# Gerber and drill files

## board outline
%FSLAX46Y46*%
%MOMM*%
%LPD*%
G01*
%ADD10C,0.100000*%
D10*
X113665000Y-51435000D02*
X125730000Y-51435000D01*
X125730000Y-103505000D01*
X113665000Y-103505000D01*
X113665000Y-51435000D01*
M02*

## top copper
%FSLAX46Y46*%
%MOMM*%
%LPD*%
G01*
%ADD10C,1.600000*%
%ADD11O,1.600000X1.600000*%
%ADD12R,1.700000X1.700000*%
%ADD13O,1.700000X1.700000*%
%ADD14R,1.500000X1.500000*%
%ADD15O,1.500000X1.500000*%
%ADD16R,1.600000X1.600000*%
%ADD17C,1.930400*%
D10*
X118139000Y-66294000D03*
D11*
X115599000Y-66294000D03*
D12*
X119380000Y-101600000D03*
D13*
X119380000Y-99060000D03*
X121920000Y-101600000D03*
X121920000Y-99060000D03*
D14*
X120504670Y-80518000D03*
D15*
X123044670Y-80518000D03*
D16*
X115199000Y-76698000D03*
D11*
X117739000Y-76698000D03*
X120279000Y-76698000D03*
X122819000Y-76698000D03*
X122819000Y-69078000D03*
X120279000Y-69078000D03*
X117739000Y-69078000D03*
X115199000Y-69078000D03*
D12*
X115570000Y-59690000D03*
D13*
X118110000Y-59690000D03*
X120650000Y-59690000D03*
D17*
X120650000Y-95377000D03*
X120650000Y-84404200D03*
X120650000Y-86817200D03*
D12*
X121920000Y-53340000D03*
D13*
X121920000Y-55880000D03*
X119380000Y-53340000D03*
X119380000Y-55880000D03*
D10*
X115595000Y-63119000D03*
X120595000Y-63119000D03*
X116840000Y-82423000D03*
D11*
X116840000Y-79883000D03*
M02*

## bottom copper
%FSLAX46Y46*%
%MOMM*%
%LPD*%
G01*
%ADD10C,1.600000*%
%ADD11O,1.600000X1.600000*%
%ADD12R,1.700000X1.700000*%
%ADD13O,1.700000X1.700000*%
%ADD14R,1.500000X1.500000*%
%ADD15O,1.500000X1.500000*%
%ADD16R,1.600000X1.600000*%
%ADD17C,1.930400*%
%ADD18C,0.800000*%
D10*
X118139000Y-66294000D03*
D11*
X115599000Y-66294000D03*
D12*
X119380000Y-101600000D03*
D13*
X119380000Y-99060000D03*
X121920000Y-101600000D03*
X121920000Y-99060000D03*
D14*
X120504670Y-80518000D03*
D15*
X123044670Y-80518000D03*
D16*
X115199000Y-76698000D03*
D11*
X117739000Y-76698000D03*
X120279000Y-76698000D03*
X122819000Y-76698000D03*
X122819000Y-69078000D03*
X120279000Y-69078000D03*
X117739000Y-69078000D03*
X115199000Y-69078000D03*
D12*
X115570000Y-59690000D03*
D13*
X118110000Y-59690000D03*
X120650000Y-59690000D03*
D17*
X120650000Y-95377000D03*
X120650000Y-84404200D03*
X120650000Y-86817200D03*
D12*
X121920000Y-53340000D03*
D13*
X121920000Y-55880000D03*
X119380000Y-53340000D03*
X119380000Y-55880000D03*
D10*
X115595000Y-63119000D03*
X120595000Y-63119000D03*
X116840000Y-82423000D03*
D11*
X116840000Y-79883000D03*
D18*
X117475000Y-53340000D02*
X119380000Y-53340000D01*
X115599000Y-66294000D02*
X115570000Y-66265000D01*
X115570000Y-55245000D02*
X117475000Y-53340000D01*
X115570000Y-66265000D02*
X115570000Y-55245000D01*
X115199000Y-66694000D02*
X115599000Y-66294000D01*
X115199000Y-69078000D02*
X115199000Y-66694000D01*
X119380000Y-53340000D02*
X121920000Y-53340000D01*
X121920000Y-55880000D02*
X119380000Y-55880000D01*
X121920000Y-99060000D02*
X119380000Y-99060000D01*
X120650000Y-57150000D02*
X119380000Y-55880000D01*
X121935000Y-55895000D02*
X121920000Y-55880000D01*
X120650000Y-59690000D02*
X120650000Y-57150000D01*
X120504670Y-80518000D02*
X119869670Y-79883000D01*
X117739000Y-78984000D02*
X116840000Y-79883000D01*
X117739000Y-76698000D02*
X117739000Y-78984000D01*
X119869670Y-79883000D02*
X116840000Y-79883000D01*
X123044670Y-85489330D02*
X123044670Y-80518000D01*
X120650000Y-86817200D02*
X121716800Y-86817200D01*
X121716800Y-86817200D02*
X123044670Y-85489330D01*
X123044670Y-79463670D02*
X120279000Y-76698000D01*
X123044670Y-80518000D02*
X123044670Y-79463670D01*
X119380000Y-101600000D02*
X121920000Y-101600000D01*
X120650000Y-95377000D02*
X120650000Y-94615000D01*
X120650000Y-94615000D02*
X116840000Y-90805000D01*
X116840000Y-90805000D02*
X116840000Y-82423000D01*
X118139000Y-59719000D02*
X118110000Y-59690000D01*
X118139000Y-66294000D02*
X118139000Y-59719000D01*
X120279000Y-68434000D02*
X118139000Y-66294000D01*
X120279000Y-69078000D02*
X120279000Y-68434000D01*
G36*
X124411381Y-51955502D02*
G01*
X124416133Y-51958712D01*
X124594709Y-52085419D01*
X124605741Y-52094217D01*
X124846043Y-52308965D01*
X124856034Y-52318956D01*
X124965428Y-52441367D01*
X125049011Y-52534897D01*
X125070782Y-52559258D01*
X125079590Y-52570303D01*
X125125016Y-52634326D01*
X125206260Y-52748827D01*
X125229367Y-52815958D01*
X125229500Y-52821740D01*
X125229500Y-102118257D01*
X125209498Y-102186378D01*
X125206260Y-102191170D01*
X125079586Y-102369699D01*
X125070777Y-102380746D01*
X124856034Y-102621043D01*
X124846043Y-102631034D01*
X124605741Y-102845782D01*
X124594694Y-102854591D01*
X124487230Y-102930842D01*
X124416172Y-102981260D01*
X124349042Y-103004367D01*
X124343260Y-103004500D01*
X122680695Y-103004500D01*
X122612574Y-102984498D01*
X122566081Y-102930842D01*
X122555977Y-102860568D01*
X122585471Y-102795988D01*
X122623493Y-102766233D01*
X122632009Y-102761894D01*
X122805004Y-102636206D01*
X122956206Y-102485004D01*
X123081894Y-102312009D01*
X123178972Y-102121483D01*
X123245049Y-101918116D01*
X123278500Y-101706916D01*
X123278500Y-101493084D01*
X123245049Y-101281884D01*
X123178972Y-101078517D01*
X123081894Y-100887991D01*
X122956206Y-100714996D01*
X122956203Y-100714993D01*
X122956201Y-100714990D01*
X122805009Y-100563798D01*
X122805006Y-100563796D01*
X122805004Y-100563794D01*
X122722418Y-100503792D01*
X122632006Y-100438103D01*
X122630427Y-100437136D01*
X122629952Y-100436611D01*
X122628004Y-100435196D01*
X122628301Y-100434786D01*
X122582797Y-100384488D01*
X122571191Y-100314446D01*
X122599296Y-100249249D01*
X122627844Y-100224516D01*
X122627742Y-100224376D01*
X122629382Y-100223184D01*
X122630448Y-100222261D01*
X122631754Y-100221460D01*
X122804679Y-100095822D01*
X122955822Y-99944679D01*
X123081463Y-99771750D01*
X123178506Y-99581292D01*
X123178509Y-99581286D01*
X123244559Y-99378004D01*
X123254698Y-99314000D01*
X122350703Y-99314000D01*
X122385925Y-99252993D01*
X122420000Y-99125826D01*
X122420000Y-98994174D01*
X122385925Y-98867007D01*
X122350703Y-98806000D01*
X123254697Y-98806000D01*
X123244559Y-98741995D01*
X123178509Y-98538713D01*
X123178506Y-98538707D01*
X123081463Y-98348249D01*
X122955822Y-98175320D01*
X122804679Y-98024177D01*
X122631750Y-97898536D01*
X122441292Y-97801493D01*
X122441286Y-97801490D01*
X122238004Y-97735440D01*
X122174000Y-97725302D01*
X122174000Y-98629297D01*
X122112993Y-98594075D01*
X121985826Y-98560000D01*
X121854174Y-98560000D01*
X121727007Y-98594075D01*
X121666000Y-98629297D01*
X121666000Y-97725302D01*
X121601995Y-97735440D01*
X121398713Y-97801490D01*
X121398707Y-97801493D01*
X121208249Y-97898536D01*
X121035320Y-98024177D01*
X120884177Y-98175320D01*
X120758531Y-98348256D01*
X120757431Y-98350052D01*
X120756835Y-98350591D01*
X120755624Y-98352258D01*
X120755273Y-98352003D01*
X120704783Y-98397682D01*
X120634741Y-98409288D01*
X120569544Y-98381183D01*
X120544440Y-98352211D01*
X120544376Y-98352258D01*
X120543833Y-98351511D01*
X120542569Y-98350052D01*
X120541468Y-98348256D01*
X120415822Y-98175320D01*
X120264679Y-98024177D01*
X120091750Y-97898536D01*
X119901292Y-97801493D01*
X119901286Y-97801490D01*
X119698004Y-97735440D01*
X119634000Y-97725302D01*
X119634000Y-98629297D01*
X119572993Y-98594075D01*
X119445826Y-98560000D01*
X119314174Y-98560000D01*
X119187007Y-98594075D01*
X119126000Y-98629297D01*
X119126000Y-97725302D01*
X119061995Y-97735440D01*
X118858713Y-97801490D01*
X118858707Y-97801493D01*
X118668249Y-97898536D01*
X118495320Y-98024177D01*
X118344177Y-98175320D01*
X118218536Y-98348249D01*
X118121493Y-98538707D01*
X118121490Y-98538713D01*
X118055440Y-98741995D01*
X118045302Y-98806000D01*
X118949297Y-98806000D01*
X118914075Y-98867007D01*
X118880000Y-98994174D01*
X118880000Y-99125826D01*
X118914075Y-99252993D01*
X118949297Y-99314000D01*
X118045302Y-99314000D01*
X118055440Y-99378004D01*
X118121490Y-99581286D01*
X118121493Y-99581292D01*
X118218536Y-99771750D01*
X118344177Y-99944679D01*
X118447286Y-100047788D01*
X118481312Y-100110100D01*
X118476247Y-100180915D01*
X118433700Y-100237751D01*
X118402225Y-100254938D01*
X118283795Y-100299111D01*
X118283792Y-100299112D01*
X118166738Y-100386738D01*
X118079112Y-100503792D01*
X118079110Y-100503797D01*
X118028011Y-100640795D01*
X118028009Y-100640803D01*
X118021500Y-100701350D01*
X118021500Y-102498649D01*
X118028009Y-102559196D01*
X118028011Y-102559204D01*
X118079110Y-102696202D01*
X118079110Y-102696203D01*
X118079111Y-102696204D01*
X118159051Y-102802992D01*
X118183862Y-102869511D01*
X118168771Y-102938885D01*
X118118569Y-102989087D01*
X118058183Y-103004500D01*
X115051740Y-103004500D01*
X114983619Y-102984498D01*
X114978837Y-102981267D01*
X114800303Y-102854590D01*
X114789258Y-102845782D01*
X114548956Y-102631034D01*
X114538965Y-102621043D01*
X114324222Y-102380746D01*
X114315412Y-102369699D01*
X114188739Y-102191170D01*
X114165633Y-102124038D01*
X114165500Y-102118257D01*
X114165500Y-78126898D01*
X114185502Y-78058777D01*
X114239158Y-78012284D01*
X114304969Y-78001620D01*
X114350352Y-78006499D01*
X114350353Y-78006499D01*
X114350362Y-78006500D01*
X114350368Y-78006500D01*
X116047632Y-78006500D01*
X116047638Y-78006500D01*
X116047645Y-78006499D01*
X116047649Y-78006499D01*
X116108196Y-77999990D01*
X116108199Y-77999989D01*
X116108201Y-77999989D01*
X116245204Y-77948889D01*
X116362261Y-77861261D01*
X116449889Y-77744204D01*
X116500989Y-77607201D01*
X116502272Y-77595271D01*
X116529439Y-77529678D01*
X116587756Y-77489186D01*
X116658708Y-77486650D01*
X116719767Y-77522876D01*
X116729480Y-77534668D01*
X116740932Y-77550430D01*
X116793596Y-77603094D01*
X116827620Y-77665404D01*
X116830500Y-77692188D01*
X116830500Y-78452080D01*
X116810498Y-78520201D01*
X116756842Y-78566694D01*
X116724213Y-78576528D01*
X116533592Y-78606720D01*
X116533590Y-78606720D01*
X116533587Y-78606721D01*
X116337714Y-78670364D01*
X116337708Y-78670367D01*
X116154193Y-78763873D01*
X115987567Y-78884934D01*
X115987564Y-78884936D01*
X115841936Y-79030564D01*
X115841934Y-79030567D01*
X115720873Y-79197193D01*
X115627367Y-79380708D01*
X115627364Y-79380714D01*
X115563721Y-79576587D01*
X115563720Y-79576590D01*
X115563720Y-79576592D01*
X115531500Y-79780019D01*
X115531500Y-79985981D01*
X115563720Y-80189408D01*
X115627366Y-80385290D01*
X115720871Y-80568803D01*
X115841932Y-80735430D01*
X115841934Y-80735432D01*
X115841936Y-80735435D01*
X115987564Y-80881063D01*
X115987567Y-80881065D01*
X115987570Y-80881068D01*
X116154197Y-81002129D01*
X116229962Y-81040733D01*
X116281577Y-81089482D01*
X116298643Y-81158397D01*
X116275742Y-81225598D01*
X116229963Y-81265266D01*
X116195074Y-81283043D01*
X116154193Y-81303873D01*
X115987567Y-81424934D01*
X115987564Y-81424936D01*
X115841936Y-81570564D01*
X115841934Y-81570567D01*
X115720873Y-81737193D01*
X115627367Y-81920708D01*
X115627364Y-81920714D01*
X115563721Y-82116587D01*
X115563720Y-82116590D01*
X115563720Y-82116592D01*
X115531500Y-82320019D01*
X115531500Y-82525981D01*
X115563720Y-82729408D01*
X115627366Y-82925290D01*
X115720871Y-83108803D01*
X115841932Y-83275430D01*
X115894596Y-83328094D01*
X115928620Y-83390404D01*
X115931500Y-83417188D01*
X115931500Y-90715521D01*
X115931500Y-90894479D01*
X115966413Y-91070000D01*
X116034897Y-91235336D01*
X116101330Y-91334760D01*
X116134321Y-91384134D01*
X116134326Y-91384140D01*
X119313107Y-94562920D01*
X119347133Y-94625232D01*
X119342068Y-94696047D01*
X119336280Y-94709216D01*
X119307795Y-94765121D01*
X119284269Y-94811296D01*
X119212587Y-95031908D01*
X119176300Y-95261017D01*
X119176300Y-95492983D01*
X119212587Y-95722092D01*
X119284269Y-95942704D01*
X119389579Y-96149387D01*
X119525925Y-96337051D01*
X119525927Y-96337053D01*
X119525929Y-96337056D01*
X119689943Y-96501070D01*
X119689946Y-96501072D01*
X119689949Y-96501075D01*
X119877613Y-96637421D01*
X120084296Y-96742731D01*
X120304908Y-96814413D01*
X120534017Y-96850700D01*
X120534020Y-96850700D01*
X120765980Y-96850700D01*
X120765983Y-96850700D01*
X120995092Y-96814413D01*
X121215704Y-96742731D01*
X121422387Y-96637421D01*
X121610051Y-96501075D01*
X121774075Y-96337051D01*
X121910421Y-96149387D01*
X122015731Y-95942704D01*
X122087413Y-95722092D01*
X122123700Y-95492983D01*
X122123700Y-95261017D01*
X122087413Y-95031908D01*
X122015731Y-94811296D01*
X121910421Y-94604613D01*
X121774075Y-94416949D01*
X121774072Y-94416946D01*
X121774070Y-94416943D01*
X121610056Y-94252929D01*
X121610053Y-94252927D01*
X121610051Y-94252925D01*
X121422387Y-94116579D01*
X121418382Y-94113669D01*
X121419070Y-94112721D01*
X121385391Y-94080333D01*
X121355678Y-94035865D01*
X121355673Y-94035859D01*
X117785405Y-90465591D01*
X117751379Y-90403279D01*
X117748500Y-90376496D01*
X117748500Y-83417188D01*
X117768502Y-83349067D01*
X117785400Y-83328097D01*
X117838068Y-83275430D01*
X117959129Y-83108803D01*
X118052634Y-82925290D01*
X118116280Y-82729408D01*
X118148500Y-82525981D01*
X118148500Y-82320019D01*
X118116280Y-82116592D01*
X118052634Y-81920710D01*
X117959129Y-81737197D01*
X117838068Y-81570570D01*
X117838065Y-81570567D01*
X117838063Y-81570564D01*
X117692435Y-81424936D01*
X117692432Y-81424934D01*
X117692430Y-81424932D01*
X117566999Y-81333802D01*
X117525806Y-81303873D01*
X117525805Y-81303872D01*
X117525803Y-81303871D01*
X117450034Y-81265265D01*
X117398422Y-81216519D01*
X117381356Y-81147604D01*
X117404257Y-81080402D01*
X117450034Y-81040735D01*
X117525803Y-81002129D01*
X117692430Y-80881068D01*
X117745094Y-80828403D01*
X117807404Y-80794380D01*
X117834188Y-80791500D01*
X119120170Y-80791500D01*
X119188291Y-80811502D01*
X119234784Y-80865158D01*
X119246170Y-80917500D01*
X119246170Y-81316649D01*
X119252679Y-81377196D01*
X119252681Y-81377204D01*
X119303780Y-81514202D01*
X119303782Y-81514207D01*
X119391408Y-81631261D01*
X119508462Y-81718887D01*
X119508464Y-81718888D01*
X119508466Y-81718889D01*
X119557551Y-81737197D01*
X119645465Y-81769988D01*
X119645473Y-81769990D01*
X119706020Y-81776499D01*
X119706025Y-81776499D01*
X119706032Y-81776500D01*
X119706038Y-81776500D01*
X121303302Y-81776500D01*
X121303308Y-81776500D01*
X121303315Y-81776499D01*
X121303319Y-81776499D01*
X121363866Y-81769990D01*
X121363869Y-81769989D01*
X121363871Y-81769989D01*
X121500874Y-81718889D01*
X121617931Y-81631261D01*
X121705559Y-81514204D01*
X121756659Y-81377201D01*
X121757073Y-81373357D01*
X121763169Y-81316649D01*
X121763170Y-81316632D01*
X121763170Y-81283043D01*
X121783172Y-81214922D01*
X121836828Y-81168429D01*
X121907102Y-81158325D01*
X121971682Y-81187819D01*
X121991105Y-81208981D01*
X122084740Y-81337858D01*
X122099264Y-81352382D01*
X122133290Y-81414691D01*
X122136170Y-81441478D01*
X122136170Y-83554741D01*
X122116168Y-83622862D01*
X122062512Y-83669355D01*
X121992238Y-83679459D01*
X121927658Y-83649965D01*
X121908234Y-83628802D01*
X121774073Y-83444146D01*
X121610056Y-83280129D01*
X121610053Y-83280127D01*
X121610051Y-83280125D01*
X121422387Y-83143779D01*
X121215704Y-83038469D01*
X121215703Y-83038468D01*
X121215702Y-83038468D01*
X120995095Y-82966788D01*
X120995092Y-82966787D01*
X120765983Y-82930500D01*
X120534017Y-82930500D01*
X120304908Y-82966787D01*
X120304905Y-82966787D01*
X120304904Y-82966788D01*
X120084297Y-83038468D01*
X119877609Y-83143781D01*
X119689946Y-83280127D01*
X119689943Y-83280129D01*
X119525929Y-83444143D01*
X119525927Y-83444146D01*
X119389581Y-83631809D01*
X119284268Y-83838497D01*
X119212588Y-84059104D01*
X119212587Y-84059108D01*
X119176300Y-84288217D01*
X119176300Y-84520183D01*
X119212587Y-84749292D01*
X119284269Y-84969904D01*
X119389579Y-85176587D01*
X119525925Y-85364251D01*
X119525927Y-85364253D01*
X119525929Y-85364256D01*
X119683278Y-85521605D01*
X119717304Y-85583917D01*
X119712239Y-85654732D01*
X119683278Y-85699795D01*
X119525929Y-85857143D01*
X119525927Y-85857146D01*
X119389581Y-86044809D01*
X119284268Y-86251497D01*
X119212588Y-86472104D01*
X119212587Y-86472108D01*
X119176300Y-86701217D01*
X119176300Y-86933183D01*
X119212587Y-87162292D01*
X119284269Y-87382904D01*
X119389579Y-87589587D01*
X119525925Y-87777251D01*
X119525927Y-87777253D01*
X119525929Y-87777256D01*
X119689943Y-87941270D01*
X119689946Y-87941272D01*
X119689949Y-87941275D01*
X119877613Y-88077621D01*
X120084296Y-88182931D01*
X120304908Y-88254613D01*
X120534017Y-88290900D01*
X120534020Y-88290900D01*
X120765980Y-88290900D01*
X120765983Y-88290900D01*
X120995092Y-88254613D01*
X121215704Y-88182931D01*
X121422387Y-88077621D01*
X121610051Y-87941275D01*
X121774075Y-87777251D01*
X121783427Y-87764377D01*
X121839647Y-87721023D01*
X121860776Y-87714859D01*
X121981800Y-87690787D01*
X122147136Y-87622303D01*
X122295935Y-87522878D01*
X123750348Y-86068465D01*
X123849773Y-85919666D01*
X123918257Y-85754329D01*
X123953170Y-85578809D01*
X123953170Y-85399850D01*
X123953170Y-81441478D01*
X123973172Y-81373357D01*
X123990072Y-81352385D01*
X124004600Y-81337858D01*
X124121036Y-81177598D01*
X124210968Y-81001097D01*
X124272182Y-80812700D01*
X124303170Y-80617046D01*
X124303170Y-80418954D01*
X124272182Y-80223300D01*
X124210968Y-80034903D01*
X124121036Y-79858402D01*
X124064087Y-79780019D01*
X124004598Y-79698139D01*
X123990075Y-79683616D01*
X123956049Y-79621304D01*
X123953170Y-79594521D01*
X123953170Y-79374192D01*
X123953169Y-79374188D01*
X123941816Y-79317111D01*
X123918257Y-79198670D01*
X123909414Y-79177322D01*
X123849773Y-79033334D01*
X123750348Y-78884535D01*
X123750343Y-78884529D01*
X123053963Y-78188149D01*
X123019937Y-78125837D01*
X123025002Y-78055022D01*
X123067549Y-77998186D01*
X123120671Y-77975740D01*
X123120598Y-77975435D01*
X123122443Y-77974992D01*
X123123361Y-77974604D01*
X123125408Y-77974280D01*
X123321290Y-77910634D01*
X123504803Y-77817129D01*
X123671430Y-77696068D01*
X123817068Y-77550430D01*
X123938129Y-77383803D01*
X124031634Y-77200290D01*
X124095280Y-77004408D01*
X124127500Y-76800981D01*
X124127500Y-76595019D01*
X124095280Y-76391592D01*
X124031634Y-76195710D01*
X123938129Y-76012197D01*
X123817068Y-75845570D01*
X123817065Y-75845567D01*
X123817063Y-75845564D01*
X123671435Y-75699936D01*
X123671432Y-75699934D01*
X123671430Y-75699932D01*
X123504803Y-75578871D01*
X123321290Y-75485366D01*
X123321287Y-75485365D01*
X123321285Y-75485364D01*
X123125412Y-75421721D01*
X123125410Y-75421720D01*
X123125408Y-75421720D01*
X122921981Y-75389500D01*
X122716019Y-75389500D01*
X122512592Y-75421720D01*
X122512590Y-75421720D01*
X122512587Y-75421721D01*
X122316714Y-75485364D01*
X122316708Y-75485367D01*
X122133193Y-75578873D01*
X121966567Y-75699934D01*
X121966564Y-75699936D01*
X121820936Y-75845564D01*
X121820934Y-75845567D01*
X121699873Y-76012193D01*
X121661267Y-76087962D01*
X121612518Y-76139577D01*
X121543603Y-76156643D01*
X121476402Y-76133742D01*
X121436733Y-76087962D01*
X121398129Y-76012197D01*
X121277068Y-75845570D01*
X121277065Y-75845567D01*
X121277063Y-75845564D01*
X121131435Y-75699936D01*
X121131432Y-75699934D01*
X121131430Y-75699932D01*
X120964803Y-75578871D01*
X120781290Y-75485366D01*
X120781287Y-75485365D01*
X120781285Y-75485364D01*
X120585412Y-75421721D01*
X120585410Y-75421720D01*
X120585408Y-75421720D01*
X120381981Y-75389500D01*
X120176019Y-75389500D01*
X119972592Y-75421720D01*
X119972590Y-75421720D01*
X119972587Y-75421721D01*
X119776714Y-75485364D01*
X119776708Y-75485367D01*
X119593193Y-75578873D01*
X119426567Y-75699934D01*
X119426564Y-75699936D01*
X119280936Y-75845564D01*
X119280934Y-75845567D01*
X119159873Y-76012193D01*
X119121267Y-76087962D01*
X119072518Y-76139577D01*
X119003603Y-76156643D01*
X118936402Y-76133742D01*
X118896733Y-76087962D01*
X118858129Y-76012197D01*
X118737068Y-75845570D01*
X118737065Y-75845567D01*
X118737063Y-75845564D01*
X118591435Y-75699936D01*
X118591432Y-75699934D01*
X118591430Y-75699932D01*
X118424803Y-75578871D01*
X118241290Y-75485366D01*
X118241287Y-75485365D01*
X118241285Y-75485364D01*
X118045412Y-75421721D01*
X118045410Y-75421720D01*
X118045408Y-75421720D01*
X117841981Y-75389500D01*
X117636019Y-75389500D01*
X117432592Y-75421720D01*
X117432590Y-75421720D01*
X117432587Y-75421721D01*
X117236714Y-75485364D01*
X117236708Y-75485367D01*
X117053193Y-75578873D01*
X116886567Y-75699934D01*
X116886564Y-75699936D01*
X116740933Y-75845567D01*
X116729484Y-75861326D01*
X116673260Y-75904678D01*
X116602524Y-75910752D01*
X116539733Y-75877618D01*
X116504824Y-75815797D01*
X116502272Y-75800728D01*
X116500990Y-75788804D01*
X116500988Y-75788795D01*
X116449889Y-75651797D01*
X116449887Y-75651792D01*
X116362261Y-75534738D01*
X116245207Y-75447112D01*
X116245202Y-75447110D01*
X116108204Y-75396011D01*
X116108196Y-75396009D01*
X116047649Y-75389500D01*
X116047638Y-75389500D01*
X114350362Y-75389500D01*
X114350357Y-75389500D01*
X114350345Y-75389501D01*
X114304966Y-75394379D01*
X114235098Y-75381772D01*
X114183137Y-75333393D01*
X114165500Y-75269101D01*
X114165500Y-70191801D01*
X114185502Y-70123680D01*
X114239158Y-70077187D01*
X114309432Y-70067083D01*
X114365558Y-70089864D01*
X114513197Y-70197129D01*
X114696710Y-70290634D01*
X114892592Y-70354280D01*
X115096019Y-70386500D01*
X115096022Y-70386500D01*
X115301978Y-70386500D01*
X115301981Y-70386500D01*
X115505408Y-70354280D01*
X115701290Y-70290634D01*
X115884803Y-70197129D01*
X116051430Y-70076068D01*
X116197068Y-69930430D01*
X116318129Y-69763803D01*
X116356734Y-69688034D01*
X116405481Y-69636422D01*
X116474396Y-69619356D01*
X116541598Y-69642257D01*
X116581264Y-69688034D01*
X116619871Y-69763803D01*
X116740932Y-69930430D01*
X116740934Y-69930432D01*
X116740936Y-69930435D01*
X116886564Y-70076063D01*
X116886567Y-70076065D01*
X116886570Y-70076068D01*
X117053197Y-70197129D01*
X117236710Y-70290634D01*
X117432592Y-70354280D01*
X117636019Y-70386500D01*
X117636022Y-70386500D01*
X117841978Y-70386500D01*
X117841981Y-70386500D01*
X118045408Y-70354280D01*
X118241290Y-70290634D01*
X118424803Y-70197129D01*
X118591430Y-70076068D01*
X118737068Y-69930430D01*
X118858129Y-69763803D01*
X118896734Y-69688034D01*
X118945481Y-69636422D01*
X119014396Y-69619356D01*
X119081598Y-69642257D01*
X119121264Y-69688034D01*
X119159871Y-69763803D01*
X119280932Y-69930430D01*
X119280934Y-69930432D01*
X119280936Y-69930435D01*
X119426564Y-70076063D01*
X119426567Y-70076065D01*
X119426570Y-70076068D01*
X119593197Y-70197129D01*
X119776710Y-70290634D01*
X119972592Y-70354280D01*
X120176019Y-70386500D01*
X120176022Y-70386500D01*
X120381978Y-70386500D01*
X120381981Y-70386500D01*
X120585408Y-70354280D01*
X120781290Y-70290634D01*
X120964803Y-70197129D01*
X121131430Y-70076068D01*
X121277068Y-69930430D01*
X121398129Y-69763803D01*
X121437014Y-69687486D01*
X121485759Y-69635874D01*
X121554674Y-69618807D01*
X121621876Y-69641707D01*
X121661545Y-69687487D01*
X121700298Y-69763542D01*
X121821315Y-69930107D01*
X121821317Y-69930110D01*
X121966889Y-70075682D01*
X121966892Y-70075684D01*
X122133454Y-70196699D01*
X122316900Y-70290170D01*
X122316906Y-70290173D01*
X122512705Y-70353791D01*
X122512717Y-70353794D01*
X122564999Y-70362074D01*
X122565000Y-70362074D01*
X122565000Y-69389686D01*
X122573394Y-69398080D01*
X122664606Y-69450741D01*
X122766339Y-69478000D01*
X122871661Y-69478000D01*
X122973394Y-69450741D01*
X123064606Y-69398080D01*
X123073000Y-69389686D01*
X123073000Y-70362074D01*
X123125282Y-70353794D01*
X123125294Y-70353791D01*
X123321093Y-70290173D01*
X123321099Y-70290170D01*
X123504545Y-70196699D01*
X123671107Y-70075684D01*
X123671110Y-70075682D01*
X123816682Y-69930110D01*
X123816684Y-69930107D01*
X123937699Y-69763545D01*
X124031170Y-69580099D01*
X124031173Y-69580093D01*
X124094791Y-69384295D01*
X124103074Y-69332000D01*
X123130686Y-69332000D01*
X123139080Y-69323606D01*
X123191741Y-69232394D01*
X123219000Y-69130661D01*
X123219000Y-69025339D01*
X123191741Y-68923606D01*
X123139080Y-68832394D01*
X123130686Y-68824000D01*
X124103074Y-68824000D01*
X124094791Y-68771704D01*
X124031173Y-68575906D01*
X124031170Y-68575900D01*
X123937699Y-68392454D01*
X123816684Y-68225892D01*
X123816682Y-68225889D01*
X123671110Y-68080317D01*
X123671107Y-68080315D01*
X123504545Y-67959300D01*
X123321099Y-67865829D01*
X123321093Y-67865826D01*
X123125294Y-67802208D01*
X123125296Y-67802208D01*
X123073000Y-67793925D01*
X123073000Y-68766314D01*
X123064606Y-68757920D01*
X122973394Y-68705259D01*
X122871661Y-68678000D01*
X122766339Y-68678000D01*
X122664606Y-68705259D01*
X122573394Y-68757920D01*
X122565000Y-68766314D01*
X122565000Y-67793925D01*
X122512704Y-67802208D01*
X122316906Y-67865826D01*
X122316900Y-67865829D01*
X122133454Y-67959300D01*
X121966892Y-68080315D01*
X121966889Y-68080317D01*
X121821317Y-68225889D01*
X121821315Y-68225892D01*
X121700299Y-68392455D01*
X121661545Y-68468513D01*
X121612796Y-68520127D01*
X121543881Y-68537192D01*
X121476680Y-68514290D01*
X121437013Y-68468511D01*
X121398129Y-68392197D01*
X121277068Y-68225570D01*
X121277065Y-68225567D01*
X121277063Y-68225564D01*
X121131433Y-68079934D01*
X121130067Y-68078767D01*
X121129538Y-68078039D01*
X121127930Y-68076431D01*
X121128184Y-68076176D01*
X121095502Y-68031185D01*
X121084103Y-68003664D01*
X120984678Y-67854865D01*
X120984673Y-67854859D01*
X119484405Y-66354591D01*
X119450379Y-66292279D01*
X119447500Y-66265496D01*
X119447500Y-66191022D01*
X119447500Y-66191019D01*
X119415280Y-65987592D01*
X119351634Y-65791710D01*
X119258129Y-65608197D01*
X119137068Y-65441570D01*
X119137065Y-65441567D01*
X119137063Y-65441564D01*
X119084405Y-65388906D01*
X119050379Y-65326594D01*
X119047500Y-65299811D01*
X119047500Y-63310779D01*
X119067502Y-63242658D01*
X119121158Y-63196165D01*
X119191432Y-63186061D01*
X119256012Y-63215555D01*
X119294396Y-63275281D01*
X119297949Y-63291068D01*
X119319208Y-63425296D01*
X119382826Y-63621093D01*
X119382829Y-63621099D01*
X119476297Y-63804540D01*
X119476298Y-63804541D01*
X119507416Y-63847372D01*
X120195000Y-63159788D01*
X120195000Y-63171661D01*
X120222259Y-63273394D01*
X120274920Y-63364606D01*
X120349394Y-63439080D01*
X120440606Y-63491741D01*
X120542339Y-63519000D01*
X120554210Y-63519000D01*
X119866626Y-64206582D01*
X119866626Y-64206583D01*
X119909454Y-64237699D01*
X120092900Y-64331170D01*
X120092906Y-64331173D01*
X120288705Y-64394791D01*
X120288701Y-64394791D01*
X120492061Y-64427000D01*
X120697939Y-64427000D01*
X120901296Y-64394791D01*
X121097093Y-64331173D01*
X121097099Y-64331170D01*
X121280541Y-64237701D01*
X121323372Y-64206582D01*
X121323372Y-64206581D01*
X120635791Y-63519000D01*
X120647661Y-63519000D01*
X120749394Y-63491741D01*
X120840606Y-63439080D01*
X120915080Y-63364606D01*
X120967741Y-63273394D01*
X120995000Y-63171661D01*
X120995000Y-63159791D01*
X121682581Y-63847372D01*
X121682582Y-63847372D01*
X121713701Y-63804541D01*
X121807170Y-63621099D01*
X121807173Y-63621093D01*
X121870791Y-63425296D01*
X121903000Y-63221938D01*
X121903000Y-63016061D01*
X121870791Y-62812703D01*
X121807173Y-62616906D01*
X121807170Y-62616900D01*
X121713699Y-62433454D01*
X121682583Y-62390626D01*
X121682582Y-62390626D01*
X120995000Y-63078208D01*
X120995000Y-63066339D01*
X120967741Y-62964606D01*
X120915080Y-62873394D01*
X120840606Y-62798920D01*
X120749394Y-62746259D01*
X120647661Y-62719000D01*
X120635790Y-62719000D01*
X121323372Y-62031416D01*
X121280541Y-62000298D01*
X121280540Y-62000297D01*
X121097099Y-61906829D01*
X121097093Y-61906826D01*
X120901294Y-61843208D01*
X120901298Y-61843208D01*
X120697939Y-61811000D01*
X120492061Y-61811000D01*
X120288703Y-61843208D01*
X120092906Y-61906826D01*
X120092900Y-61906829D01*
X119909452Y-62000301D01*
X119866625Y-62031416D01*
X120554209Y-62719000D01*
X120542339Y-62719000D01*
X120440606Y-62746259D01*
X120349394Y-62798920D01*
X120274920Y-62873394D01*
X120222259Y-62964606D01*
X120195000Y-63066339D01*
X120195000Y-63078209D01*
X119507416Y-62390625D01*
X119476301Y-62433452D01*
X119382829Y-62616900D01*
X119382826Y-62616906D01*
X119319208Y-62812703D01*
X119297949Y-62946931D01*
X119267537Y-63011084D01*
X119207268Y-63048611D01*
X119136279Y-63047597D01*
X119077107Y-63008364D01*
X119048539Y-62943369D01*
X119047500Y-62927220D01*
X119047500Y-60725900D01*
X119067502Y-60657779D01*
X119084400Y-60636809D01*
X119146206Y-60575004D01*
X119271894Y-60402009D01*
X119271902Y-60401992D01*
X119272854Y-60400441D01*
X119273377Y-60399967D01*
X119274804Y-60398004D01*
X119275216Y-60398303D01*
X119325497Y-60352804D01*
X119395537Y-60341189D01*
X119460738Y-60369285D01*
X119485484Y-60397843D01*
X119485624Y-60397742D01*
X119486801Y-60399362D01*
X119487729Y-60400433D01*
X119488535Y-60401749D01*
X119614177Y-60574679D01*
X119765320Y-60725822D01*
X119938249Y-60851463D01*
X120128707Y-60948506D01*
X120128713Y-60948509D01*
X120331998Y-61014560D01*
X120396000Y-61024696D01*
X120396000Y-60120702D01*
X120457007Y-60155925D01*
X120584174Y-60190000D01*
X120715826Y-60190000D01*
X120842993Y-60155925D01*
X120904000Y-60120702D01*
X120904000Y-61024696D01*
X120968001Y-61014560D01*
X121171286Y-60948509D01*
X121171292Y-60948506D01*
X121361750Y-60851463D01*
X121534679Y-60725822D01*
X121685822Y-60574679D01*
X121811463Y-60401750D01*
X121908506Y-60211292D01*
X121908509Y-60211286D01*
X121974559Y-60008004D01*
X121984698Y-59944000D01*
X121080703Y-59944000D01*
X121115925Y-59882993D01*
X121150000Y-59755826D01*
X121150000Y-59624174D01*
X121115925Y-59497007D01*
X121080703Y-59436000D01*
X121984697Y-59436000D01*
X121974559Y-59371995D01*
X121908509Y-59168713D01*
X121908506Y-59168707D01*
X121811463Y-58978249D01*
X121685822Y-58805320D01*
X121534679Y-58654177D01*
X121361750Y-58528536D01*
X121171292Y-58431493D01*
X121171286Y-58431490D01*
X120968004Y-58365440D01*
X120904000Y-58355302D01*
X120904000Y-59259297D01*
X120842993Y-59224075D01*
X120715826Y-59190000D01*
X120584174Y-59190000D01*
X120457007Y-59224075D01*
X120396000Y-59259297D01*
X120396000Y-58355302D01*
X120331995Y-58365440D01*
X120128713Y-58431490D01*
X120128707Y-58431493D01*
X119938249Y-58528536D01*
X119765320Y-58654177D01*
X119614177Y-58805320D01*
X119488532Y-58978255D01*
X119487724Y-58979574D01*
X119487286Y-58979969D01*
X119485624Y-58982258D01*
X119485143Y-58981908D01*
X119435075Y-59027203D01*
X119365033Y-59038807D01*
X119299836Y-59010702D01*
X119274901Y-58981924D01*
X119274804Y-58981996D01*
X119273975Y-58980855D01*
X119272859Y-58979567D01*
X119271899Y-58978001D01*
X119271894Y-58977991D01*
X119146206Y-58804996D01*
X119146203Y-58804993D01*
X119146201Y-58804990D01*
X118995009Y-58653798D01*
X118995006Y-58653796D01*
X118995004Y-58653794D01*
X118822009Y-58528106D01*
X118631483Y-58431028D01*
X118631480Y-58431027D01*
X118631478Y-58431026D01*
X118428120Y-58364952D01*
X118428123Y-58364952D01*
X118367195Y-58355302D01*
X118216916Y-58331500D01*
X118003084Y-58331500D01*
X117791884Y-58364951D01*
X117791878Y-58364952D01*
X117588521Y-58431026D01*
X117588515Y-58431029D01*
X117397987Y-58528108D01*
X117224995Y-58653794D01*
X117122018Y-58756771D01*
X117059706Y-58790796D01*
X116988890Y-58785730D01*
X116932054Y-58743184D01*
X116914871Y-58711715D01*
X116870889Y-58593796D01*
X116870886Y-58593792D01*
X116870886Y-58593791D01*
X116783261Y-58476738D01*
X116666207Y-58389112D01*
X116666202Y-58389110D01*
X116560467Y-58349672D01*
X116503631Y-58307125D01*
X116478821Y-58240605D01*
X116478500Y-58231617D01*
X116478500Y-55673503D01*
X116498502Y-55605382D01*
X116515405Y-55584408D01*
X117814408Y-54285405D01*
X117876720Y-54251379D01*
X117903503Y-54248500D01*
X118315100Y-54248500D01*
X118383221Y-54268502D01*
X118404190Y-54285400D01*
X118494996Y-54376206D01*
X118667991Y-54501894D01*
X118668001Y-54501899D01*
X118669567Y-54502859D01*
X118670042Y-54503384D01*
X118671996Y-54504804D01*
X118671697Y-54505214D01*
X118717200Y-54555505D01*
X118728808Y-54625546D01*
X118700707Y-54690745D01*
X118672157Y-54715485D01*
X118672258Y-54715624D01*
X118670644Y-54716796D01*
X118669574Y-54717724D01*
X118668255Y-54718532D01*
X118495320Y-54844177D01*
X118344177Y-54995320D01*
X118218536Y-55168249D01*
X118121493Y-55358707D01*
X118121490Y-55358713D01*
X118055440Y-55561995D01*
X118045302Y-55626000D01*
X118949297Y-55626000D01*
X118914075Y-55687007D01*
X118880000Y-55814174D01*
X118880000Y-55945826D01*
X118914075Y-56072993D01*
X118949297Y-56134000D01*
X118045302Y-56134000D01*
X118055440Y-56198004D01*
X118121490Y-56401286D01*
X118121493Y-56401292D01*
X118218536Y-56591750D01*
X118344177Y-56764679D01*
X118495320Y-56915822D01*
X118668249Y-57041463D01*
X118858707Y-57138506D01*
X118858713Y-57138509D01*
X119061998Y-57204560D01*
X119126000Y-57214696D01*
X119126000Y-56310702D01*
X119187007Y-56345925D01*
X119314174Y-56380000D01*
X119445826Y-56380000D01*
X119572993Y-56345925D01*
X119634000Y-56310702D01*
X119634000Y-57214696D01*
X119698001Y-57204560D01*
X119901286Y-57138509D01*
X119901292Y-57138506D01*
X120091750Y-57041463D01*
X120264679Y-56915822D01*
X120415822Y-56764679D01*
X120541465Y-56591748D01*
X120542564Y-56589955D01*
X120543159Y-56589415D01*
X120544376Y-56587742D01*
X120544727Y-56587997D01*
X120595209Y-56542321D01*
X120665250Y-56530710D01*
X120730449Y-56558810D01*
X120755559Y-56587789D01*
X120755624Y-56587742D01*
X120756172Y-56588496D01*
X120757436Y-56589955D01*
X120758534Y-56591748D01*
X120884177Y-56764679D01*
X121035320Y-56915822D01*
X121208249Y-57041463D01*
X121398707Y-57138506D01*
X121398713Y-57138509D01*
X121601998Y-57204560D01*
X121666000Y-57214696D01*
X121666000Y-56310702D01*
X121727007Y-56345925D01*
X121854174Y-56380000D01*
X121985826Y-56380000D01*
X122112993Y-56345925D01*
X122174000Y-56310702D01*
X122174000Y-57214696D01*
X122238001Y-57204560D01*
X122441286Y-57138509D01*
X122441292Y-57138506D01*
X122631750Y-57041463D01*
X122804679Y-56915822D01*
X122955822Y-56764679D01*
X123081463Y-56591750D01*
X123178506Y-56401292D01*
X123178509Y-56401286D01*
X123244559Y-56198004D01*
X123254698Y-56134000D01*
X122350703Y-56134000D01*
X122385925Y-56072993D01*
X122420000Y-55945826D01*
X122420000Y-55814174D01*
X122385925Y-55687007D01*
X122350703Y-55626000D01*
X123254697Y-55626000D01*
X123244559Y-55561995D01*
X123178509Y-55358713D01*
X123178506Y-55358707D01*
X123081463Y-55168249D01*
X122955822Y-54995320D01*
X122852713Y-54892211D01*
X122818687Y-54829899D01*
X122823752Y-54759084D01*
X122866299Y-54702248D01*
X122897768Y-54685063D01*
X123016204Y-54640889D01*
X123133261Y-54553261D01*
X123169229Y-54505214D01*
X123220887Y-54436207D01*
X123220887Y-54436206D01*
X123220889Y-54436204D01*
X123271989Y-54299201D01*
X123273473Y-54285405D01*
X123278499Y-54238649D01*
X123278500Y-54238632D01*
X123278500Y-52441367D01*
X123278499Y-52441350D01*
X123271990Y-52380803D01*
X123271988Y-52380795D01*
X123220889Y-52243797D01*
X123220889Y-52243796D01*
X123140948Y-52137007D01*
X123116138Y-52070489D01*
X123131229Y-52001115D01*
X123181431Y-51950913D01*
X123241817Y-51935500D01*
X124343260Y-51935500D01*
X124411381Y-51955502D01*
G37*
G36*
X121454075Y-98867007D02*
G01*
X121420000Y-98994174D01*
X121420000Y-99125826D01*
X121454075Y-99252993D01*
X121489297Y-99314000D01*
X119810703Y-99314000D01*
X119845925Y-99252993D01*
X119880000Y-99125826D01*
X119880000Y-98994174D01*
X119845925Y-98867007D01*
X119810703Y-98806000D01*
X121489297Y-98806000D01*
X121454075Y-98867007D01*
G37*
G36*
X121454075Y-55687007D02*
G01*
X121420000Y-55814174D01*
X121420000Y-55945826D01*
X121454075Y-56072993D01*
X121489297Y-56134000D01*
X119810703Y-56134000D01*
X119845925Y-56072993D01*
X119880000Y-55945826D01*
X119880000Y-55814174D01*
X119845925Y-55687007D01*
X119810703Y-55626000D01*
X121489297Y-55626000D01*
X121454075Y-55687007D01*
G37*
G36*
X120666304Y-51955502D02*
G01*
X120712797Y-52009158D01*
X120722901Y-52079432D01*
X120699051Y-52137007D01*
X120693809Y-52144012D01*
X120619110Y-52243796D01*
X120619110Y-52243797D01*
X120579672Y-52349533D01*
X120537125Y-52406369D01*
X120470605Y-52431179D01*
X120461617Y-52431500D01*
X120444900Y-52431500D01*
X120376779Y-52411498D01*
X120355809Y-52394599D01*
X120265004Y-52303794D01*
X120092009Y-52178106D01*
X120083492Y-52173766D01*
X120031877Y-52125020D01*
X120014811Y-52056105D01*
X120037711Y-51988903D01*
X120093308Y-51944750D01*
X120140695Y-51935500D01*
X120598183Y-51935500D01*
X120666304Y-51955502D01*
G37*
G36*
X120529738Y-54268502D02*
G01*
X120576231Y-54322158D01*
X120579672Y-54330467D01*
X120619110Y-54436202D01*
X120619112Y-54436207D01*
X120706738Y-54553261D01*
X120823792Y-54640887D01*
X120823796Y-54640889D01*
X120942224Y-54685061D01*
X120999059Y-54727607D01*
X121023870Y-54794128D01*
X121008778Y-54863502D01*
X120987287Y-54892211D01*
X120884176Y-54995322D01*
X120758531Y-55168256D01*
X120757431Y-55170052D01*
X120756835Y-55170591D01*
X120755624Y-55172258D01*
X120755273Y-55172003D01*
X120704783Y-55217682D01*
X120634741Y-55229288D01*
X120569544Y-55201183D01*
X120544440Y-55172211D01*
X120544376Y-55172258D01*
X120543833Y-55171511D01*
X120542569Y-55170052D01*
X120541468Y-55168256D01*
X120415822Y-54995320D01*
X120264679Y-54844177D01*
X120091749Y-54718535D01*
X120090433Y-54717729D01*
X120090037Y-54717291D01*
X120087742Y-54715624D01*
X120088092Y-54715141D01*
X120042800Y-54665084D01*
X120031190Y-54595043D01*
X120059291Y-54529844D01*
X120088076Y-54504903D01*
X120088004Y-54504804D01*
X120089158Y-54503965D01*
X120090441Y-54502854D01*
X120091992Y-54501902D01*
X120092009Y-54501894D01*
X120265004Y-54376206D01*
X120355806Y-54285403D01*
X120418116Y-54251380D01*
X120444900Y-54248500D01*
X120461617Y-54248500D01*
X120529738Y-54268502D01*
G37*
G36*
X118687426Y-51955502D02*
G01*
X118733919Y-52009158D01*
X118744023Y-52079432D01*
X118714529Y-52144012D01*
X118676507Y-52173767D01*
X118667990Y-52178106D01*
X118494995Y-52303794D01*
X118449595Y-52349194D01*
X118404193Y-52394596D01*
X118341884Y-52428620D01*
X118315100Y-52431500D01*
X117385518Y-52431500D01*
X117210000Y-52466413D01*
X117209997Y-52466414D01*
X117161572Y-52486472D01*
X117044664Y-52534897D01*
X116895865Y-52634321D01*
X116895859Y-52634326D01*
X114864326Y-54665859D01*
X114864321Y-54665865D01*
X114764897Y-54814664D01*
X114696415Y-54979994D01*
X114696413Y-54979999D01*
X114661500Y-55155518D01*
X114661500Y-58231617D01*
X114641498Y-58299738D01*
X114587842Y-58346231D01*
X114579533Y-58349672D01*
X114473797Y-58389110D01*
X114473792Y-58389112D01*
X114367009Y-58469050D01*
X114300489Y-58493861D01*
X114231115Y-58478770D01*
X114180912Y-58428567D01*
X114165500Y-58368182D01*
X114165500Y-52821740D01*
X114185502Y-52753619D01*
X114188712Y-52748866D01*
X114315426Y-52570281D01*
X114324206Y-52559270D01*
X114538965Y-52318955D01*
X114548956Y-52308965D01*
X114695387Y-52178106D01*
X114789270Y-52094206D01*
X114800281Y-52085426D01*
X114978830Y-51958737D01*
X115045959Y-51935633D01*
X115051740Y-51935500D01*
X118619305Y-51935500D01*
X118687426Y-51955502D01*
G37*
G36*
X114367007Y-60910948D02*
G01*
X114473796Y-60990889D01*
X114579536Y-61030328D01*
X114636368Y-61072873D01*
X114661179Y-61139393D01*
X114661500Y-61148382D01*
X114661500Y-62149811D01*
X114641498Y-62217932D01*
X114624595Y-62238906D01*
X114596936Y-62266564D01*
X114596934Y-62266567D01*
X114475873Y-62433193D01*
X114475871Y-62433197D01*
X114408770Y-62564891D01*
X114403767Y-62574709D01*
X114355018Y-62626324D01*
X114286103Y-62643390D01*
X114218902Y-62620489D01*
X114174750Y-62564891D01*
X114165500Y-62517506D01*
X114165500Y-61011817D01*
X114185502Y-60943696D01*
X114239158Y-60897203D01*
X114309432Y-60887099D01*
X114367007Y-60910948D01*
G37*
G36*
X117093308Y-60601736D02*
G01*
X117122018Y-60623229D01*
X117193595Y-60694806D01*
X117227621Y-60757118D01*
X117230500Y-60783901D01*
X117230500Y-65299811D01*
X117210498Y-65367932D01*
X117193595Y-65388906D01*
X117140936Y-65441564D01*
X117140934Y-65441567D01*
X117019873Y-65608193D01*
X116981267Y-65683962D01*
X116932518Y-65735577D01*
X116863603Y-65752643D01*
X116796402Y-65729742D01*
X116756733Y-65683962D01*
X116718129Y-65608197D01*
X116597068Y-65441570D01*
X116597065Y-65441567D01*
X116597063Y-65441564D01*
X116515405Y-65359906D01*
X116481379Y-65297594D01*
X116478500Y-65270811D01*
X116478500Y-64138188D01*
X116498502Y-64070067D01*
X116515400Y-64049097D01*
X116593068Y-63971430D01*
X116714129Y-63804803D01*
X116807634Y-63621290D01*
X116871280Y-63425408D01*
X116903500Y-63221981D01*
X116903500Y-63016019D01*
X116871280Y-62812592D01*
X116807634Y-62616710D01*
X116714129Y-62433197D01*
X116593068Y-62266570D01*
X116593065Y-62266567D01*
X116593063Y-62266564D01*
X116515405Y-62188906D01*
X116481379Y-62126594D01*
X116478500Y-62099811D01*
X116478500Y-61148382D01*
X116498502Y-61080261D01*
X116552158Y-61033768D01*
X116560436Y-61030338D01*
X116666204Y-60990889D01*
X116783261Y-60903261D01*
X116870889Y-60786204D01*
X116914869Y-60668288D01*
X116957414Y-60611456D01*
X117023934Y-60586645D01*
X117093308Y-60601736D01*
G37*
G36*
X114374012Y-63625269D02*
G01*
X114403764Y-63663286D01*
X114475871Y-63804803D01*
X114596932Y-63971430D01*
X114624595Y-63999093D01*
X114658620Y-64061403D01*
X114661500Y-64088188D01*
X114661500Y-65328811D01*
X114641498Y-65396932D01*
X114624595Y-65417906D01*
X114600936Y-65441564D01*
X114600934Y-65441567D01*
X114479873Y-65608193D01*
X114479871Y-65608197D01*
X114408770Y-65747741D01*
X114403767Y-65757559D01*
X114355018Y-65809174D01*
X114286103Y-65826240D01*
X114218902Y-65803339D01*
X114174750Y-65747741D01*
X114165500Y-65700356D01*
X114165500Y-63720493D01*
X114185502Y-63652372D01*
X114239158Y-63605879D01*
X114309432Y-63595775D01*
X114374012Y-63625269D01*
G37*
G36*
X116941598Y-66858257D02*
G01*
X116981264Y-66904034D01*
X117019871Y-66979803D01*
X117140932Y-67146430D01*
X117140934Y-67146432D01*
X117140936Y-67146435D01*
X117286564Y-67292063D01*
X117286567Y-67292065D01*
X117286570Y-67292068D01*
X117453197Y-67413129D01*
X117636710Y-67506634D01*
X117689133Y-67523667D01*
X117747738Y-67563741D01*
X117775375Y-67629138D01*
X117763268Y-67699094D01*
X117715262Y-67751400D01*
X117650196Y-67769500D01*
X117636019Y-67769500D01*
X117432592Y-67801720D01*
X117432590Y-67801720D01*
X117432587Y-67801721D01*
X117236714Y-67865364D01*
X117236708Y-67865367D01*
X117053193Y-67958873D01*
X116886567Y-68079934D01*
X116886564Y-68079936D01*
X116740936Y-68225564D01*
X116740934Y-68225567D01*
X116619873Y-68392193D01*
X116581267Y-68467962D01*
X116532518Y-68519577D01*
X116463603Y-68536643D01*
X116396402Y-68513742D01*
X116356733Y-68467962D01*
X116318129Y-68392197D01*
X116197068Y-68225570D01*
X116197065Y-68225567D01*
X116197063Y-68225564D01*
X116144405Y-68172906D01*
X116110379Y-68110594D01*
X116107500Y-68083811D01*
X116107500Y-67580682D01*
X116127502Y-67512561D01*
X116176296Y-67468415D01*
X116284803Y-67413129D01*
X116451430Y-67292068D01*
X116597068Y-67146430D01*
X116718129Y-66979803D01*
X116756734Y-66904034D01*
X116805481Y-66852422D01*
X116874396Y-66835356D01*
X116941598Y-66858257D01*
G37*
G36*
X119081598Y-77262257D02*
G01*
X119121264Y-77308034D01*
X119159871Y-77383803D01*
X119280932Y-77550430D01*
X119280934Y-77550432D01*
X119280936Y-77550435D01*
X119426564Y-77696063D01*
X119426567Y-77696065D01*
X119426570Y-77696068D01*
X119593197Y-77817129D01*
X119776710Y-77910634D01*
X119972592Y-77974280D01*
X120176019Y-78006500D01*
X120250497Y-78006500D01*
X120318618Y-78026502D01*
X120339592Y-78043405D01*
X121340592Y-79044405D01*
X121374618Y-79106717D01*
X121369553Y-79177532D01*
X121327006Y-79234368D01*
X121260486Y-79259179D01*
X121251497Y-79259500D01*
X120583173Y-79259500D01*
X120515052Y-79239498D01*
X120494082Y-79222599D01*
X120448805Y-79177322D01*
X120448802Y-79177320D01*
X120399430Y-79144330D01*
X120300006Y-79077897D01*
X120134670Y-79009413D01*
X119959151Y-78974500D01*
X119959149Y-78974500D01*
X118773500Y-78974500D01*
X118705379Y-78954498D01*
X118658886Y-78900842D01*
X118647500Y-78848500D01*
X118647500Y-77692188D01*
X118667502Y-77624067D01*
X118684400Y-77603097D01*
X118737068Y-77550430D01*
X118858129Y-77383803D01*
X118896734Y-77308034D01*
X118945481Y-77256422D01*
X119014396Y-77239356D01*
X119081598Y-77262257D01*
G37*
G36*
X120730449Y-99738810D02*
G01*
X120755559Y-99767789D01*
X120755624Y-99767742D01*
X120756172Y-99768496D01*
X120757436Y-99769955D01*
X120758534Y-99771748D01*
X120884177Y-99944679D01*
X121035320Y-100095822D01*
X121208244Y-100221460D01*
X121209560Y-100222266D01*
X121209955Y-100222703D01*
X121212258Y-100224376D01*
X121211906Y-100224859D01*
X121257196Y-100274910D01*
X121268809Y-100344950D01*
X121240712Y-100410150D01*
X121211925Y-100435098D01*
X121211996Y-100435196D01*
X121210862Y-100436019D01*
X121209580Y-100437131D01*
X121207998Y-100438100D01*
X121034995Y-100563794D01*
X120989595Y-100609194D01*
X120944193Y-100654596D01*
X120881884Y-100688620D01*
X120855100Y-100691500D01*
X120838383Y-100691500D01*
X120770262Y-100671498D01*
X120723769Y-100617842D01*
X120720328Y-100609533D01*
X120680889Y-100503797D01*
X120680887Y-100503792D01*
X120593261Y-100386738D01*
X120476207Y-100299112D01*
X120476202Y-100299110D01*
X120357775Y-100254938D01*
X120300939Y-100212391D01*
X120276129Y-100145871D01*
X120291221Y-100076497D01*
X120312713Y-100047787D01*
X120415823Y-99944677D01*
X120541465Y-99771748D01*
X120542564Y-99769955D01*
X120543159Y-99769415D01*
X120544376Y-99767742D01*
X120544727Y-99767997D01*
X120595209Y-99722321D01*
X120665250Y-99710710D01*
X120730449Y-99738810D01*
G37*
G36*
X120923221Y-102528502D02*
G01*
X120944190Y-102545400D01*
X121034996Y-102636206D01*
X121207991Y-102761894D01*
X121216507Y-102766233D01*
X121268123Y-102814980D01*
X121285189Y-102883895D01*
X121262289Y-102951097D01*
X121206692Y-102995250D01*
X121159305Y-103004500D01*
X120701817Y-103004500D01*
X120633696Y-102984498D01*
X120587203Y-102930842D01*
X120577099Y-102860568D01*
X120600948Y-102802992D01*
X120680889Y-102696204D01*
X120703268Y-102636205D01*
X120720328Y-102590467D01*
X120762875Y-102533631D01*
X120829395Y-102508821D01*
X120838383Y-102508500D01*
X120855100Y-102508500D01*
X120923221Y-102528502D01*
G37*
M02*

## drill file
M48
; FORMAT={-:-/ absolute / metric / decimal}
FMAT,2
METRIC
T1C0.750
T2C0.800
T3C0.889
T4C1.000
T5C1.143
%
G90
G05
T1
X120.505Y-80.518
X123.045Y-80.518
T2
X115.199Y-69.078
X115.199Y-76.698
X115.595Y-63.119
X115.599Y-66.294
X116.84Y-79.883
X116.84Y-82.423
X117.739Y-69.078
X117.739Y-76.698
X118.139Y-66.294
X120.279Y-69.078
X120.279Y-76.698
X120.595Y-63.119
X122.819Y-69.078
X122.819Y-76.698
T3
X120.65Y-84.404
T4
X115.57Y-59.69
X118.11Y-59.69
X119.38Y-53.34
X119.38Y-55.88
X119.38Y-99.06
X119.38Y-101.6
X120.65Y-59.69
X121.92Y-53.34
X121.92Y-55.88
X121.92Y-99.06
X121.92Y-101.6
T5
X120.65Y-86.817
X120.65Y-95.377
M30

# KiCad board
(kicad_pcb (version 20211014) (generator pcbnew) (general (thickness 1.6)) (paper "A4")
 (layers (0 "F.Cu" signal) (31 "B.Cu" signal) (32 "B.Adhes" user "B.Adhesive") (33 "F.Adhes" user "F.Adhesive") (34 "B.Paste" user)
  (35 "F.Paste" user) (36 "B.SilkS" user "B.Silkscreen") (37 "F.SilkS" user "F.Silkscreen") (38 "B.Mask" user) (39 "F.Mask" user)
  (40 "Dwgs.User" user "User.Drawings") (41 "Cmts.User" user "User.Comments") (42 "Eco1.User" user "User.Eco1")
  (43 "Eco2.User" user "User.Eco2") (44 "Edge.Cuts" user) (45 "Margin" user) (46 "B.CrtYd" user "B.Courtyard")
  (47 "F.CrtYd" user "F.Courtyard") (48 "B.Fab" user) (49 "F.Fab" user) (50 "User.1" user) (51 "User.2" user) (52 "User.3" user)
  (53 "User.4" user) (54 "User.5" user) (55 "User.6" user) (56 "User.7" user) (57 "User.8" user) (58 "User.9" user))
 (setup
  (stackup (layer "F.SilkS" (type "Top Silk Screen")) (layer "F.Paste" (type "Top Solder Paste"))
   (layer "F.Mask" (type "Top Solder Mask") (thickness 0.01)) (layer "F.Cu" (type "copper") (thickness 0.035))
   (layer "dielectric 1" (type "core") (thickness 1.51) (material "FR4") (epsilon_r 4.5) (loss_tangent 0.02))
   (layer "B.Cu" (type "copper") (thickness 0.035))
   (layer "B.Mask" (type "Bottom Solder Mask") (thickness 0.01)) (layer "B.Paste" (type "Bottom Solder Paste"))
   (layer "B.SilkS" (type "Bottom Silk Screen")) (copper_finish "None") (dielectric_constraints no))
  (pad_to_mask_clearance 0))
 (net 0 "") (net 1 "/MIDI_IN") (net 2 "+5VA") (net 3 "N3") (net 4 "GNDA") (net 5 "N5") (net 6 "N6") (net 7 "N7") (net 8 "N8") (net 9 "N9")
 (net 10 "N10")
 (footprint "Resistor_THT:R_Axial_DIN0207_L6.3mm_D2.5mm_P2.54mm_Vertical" (layer "F.Cu") (at 118.139 66.294 180)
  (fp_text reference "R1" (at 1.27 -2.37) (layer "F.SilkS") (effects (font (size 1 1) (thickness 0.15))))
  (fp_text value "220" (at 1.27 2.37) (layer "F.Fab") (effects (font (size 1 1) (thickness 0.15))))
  (pad "1" thru_hole circle (at 0 0 180) (size 1.6 1.6) (drill 0.8) (layers *.Cu *.Mask) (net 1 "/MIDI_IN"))
  (pad "2" thru_hole oval (at 2.54 0 180) (size 1.6 1.6) (drill 0.8) (layers *.Cu *.Mask) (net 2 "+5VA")))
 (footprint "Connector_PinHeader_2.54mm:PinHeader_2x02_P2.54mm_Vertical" (layer "F.Cu") (at 119.38 101.6 90)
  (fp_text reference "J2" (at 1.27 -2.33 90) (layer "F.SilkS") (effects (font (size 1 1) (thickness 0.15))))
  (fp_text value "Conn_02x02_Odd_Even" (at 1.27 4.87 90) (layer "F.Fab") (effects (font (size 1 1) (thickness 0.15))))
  (pad "1" thru_hole rect (at 0 0 90) (size 1.7 1.7) (drill 1) (layers *.Cu *.Mask) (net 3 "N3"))
  (pad "2" thru_hole oval (at 2.54 0 90) (size 1.7 1.7) (drill 1) (layers *.Cu *.Mask) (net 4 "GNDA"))
  (pad "3" thru_hole oval (at 0 2.54 90) (size 1.7 1.7) (drill 1) (layers *.Cu *.Mask) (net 3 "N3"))
  (pad "4" thru_hole oval (at 2.54 2.54 90) (size 1.7 1.7) (drill 1) (layers *.Cu *.Mask) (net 4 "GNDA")))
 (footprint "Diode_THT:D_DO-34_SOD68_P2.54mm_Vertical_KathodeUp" (layer "F.Cu") (at 120.50467 80.518)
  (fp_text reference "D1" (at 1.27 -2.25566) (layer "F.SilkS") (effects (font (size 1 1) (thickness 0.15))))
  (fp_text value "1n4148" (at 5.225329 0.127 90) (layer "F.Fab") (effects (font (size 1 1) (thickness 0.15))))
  (pad "1" thru_hole rect (at 0 0) (size 1.5 1.5) (drill 0.75) (layers *.Cu *.Mask) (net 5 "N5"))
  (pad "2" thru_hole oval (at 2.54 0) (size 1.5 1.5) (drill 0.75) (layers *.Cu *.Mask) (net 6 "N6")))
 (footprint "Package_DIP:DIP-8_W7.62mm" (layer "F.Cu") (at 115.199 76.698 90)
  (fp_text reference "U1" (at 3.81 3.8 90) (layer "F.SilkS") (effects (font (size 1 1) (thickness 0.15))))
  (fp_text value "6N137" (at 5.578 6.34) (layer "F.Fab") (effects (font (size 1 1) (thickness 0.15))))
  (pad "1" thru_hole rect (at 0 0 90) (size 1.6 1.6) (drill 0.8) (layers *.Cu *.Mask) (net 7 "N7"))
  (pad "2" thru_hole oval (at 0 2.54 90) (size 1.6 1.6) (drill 0.8) (layers *.Cu *.Mask) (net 5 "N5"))
  (pad "3" thru_hole oval (at 0 5.08 90) (size 1.6 1.6) (drill 0.8) (layers *.Cu *.Mask) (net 6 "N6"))
  (pad "4" thru_hole oval (at 0 7.62 90) (size 1.6 1.6) (drill 0.8) (layers *.Cu *.Mask))
  (pad "5" thru_hole oval (at 7.62 7.62 90) (size 1.6 1.6) (drill 0.8) (layers *.Cu *.Mask) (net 4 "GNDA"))
  (pad "6" thru_hole oval (at 7.62 5.08 90) (size 1.6 1.6) (drill 0.8) (layers *.Cu *.Mask) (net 1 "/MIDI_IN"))
  (pad "7" thru_hole oval (at 7.62 2.54 90) (size 1.6 1.6) (drill 0.8) (layers *.Cu *.Mask) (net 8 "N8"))
  (pad "8" thru_hole oval (at 7.62 0 90) (size 1.6 1.6) (drill 0.8) (layers *.Cu *.Mask) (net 2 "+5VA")))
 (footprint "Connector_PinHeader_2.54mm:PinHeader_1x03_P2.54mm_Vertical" (layer "F.Cu") (at 115.57 59.69 90)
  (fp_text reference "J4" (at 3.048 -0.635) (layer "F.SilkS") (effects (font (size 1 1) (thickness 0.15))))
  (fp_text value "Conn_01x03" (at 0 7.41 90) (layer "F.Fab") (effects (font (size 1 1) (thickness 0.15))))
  (pad "1" thru_hole rect (at 0 0 90) (size 1.7 1.7) (drill 1) (layers *.Cu *.Mask) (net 2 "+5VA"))
  (pad "2" thru_hole oval (at 0 2.54 90) (size 1.7 1.7) (drill 1) (layers *.Cu *.Mask) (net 1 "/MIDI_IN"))
  (pad "3" thru_hole oval (at 0 5.08 90) (size 1.7 1.7) (drill 1) (layers *.Cu *.Mask) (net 4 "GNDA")))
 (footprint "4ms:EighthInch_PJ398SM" (layer "F.Cu") (at 120.65 90.17 90)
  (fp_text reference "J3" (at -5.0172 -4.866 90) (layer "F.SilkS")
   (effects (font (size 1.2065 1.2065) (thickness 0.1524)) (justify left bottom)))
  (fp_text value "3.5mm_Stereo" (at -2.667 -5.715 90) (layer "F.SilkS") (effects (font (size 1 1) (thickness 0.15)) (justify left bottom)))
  (pad "1" thru_hole circle locked (at -5.207 0 90) (size 1.9304 1.9304) (drill 1.143) (layers *.Cu *.Mask) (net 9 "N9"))
  (pad "2" thru_hole circle locked (at 5.7658 0 90) (size 1.9304 1.9304) (drill 0.889) (layers *.Cu *.Mask) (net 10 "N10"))
  (pad "3" thru_hole circle locked (at 3.3528 0 90) (size 1.9304 1.9304) (drill 1.143) (layers *.Cu *.Mask) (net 6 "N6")))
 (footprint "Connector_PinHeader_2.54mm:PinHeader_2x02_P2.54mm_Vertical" (layer "F.Cu") (at 121.92 53.34 -90)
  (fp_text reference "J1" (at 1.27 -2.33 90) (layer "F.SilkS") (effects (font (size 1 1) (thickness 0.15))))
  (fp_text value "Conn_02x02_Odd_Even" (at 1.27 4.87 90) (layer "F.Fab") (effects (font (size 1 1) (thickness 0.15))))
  (pad "1" thru_hole rect (at 0 0 270) (size 1.7 1.7) (drill 1) (layers *.Cu *.Mask) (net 2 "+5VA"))
  (pad "2" thru_hole oval (at 2.54 0 270) (size 1.7 1.7) (drill 1) (layers *.Cu *.Mask) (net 4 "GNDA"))
  (pad "3" thru_hole oval (at 0 2.54 270) (size 1.7 1.7) (drill 1) (layers *.Cu *.Mask) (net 2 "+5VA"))
  (pad "4" thru_hole oval (at 2.54 2.54 270) (size 1.7 1.7) (drill 1) (layers *.Cu *.Mask) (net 4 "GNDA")))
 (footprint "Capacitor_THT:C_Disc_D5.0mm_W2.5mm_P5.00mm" (layer "F.Cu") (at 115.595 63.119)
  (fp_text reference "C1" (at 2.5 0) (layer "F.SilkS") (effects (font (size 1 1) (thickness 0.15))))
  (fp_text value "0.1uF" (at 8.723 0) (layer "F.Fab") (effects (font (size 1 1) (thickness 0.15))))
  (pad "1" thru_hole circle (at 0 0) (size 1.6 1.6) (drill 0.8) (layers *.Cu *.Mask) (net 2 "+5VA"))
  (pad "2" thru_hole circle (at 5 0) (size 1.6 1.6) (drill 0.8) (layers *.Cu *.Mask) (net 4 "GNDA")))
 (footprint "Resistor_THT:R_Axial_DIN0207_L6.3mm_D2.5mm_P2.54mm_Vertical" (layer "F.Cu") (at 116.84 82.423 90)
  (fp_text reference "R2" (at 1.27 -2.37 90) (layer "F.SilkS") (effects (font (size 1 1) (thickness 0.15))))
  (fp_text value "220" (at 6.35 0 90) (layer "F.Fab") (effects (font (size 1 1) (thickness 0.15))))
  (pad "1" thru_hole circle (at 0 0 90) (size 1.6 1.6) (drill 0.8) (layers *.Cu *.Mask) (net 9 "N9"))
  (pad "2" thru_hole oval (at 2.54 0 90) (size 1.6 1.6) (drill 0.8) (layers *.Cu *.Mask) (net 5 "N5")))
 (gr_rect (start 113.665 51.435) (end 125.73 103.505) (layer "Edge.Cuts") (width 0.1) (fill none))
 (segment (start 117.475 53.34) (end 119.38 53.34) (width 0.8) (layer "B.Cu") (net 2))
 (segment (start 115.599 66.294) (end 115.57 66.265) (width 0.8) (layer "B.Cu") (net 2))
 (segment (start 115.57 55.245) (end 117.475 53.34) (width 0.8) (layer "B.Cu") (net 2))
 (segment (start 115.57 66.265) (end 115.57 55.245) (width 0.8) (layer "B.Cu") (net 2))
 (segment (start 115.199 66.694) (end 115.599 66.294) (width 0.8) (layer "B.Cu") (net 2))
 (segment (start 115.199 69.078) (end 115.199 66.694) (width 0.8) (layer "B.Cu") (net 2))
 (segment (start 119.38 53.34) (end 121.92 53.34) (width 0.8) (layer "B.Cu") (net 2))
 (segment (start 121.92 55.88) (end 119.38 55.88) (width 0.8) (layer "B.Cu") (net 4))
 (segment (start 121.92 99.06) (end 119.38 99.06) (width 0.8) (layer "B.Cu") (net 4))
 (segment (start 120.65 57.15) (end 119.38 55.88) (width 0.8) (layer "B.Cu") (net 4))
 (segment (start 121.935 55.895) (end 121.92 55.88) (width 0.8) (layer "B.Cu") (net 4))
 (segment (start 120.65 59.69) (end 120.65 57.15) (width 0.8) (layer "B.Cu") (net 4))
 (segment (start 120.50467 80.518) (end 119.86967 79.883) (width 0.8) (layer "B.Cu") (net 5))
 (segment (start 117.739 78.984) (end 116.84 79.883) (width 0.8) (layer "B.Cu") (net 5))
 (segment (start 117.739 76.698) (end 117.739 78.984) (width 0.8) (layer "B.Cu") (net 5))
 (segment (start 119.86967 79.883) (end 116.84 79.883) (width 0.8) (layer "B.Cu") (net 5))
 (segment (start 123.04467 85.48933) (end 123.04467 80.518) (width 0.8) (layer "B.Cu") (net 6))
 (segment (start 120.65 86.8172) (end 121.7168 86.8172) (width 0.8) (layer "B.Cu") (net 6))
 (segment (start 121.7168 86.8172) (end 123.04467 85.48933) (width 0.8) (layer "B.Cu") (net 6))
 (segment (start 123.04467 79.46367) (end 120.279 76.698) (width 0.8) (layer "B.Cu") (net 6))
 (segment (start 123.04467 80.518) (end 123.04467 79.46367) (width 0.8) (layer "B.Cu") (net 6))
 (segment (start 119.38 101.6) (end 121.92 101.6) (width 0.8) (layer "B.Cu") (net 3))
 (segment (start 120.65 95.377) (end 120.65 94.615) (width 0.8) (layer "B.Cu") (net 9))
 (segment (start 120.65 94.615) (end 116.84 90.805) (width 0.8) (layer "B.Cu") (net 9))
 (segment (start 116.84 90.805) (end 116.84 82.423) (width 0.8) (layer "B.Cu") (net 9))
 (segment (start 118.139 59.719) (end 118.11 59.69) (width 0.8) (layer "B.Cu") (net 1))
 (segment (start 118.139 66.294) (end 118.139 59.719) (width 0.8) (layer "B.Cu") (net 1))
 (segment (start 120.279 68.434) (end 118.139 66.294) (width 0.8) (layer "B.Cu") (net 1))
 (segment (start 120.279 69.078) (end 120.279 68.434) (width 0.8) (layer "B.Cu") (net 1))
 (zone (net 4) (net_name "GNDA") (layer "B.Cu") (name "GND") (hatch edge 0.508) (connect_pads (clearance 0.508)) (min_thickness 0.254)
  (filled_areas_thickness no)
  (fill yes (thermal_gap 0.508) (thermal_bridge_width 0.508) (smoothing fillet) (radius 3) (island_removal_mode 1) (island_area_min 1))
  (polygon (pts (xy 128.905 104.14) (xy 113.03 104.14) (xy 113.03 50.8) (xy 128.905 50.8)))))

